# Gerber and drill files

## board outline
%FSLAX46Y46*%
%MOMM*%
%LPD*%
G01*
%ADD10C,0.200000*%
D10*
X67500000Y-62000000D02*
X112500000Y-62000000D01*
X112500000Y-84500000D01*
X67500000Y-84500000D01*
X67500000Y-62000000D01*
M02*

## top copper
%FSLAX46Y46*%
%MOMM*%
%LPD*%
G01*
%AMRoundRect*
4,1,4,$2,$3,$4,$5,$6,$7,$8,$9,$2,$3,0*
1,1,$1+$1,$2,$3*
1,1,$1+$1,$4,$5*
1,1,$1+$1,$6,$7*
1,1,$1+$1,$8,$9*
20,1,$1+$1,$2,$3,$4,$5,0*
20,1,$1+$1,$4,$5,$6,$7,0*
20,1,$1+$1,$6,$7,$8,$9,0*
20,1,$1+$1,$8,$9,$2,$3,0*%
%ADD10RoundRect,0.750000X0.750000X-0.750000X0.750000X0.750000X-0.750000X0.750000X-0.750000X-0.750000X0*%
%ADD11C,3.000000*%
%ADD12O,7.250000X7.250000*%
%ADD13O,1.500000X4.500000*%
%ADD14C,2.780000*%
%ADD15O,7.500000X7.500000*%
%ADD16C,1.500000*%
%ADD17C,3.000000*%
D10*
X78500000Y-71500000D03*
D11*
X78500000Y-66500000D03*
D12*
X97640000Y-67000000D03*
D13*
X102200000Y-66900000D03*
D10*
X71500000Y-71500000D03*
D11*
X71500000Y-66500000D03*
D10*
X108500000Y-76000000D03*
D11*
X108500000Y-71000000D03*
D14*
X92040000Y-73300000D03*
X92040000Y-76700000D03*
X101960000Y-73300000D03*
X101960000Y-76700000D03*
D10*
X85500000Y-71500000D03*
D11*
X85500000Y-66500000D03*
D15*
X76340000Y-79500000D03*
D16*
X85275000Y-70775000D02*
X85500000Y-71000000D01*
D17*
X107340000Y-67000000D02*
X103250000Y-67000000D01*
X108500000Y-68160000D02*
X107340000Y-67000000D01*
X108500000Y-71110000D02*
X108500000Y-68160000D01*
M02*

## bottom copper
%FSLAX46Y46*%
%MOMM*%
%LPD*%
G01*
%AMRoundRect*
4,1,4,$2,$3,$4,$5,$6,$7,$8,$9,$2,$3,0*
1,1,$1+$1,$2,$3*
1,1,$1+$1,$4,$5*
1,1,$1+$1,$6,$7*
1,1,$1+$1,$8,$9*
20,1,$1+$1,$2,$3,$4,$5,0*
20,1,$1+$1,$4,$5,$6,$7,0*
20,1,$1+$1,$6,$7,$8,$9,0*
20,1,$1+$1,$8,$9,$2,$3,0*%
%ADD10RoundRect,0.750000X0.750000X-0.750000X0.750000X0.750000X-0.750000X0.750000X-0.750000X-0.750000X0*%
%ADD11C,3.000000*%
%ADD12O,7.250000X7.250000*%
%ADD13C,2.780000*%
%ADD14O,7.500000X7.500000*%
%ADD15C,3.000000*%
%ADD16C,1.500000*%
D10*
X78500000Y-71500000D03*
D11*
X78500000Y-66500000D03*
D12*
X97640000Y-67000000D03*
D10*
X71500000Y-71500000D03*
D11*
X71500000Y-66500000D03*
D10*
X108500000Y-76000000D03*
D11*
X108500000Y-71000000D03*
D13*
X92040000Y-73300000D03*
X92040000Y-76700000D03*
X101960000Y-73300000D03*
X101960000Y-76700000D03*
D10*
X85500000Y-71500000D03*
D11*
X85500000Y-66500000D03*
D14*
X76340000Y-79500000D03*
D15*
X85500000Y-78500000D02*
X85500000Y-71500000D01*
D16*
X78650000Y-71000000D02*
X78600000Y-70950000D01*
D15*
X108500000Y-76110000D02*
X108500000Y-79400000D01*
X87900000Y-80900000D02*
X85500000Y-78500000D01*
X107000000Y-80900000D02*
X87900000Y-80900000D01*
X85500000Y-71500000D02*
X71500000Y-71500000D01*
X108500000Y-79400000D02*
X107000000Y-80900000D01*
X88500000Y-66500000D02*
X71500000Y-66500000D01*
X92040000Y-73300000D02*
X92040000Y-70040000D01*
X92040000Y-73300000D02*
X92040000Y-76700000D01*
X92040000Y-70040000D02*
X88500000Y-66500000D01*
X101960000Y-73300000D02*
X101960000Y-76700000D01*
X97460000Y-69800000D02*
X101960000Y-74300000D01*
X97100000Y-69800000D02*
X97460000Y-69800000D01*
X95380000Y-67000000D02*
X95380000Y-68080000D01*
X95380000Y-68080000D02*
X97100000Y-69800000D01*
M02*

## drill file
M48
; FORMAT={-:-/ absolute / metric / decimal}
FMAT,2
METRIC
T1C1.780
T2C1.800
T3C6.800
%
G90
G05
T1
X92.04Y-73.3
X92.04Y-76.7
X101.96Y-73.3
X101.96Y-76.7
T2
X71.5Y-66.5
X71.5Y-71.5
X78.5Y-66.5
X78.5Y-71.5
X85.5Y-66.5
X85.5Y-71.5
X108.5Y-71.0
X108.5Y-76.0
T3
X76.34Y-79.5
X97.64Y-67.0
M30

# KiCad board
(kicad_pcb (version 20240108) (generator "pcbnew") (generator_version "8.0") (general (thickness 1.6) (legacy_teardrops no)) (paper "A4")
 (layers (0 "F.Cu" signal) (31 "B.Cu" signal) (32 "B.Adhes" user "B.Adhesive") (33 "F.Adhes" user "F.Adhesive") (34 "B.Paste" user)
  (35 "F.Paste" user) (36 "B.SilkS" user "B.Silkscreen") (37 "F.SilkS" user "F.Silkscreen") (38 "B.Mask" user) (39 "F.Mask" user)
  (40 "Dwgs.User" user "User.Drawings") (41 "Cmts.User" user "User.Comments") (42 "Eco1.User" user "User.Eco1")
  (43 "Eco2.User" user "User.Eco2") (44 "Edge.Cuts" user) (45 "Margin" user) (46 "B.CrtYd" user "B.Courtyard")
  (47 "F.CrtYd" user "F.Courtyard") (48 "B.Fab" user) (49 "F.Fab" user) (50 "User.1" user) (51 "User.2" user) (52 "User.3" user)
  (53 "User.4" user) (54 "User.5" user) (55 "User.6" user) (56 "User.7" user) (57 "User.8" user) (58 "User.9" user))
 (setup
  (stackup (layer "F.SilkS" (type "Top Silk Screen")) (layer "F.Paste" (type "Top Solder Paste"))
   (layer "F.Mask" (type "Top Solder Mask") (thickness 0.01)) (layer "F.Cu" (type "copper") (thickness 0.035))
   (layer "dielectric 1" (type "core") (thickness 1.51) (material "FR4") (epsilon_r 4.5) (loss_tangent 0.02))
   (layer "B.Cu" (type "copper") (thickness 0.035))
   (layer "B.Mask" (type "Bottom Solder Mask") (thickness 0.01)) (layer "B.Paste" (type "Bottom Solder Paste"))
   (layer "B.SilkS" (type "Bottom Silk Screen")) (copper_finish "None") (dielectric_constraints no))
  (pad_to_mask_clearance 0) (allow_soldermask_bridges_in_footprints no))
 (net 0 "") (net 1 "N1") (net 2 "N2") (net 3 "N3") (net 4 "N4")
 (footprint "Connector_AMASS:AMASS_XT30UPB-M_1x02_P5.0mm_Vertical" (layer "F.Cu") (at 78.5 71.5 90)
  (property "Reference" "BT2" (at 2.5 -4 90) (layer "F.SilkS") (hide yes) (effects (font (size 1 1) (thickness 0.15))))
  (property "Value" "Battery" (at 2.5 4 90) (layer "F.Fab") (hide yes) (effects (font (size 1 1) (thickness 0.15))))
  (pad "1" thru_hole roundrect (at 0 0 90) (size 3 3) (drill 1.8) (layers "*.Cu" "*.Mask") (remove_unused_layers no) (roundrect_rratio 0.25)
   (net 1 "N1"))
  (pad "2" thru_hole circle (at 5 0 90) (size 3 3) (drill 1.8) (layers "*.Cu" "*.Mask") (remove_unused_layers no) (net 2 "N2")))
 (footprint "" (layer "F.Cu") (at 97.64 67)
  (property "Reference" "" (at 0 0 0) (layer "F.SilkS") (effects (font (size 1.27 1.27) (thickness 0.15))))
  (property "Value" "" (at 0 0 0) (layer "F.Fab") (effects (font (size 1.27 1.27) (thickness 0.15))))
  (pad "" thru_hole oval (at 0 0 270) (size 7.25 7.25) (drill 6.8) (layers "*.Cu" "*.Mask") (remove_unused_layers no)))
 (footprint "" (layer "F.Cu") (at 102.2 66.9)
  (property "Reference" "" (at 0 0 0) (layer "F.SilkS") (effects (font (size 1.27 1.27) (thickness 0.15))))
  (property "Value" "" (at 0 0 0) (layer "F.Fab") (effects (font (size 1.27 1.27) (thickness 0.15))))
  (pad "2" smd oval (at 0 0) (size 1.5 4.5) (layers "F.Cu" "F.Paste" "F.Mask") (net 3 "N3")))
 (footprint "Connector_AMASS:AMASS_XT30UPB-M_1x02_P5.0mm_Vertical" (layer "F.Cu") (at 71.5 71.5 90)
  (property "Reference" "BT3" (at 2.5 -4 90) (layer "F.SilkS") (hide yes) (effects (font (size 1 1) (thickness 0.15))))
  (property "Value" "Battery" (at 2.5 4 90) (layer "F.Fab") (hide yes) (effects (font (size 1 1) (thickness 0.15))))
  (pad "1" thru_hole roundrect (at 0 0 90) (size 3 3) (drill 1.8) (layers "*.Cu" "*.Mask") (remove_unused_layers no) (roundrect_rratio 0.25)
   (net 1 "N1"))
  (pad "2" thru_hole circle (at 5 0 90) (size 3 3) (drill 1.8) (layers "*.Cu" "*.Mask") (remove_unused_layers no) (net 2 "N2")))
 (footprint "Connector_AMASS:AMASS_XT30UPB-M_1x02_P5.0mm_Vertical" (layer "F.Cu") (at 108.5 76 90)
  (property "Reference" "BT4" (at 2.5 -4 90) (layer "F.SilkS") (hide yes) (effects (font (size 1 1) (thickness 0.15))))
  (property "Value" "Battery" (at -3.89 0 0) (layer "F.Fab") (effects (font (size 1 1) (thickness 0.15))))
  (pad "1" thru_hole roundrect (at 0 0 90) (size 3 3) (drill 1.8) (layers "*.Cu" "*.Mask") (remove_unused_layers no) (roundrect_rratio 0.25)
   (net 1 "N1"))
  (pad "2" thru_hole circle (at 5 0 90) (size 3 3) (drill 1.8) (layers "*.Cu" "*.Mask") (remove_unused_layers no) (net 3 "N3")))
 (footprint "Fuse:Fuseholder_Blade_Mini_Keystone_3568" (layer "F.Cu") (at 92.04 73.3)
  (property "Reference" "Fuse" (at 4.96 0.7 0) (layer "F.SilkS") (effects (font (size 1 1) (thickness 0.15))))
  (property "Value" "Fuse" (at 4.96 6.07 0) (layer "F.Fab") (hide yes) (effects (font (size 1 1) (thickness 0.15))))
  (pad "1" thru_hole circle (at 0 0) (size 2.78 2.78) (drill 1.78) (layers "*.Cu" "*.Mask") (remove_unused_layers no) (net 2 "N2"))
  (pad "1" thru_hole circle (at 0 3.4) (size 2.78 2.78) (drill 1.78) (layers "*.Cu" "*.Mask") (remove_unused_layers no) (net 2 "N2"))
  (pad "2" thru_hole circle (at 9.92 0) (size 2.78 2.78) (drill 1.78) (layers "*.Cu" "*.Mask") (remove_unused_layers no) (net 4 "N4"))
  (pad "2" thru_hole circle (at 9.92 3.4) (size 2.78 2.78) (drill 1.78) (layers "*.Cu" "*.Mask") (remove_unused_layers no) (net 4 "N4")))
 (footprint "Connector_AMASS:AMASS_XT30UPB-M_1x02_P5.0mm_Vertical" (layer "F.Cu") (at 85.5 71.5 90)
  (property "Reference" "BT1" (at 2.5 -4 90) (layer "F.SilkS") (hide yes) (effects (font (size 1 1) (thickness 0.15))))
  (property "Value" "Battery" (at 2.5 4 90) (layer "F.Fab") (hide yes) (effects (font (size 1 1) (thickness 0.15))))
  (pad "1" thru_hole roundrect (at 0 0 90) (size 3 3) (drill 1.8) (layers "*.Cu" "*.Mask") (remove_unused_layers no) (roundrect_rratio 0.25)
   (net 1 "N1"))
  (pad "2" thru_hole circle (at 5 0 90) (size 3 3) (drill 1.8) (layers "*.Cu" "*.Mask") (remove_unused_layers no) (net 2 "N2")))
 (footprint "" (layer "F.Cu") (at 76.34 79.5)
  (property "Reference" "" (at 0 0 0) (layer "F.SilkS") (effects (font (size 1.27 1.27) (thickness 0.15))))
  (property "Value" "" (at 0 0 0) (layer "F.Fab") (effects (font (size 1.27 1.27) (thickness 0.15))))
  (pad "2" thru_hole oval (at 0 0 270) (size 7.5 7.5) (drill 6.8) (layers "*.Cu" "*.Mask") (remove_unused_layers no)))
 (gr_rect (start 67.5 62) (end 112.5 84.5) (stroke (width 0.2) (type default)) (fill none) (layer "Edge.Cuts"))
 (segment (start 85.275 70.775) (end 85.5 71) (width 1.5) (layer "F.Cu") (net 1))
 (segment (start 85.5 78.5) (end 85.5 71.5) (width 3) (layer "B.Cu") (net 1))
 (segment (start 78.65 71) (end 78.6 70.95) (width 1.5) (layer "B.Cu") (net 1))
 (segment (start 108.5 76.11) (end 108.5 79.4) (width 3) (layer "B.Cu") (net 1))
 (segment (start 87.9 80.9) (end 85.5 78.5) (width 3) (layer "B.Cu") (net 1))
 (segment (start 107 80.9) (end 87.9 80.9) (width 3) (layer "B.Cu") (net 1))
 (segment (start 85.5 71.5) (end 71.5 71.5) (width 3) (layer "B.Cu") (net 1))
 (segment (start 108.5 79.4) (end 107 80.9) (width 3) (layer "B.Cu") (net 1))
 (segment (start 88.5 66.5) (end 71.5 66.5) (width 3) (layer "B.Cu") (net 2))
 (segment (start 92.04 73.3) (end 92.04 70.04) (width 3) (layer "B.Cu") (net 2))
 (segment (start 92.04 73.3) (end 92.04 76.7) (width 3) (layer "B.Cu") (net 2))
 (segment (start 92.04 70.04) (end 88.5 66.5) (width 3) (layer "B.Cu") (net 2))
 (segment (start 101.96 73.3) (end 101.96 76.7) (width 3) (layer "B.Cu") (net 4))
 (segment (start 97.46 69.8) (end 101.96 74.3) (width 3) (layer "B.Cu") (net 4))
 (segment (start 97.1 69.8) (end 97.46 69.8) (width 3) (layer "B.Cu") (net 4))
 (segment (start 95.38 67) (end 95.38 68.08) (width 3) (layer "B.Cu") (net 4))
 (segment (start 95.38 68.08) (end 97.1 69.8) (width 3) (layer "B.Cu") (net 4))
 (segment (start 107.34 67) (end 103.25 67) (width 3) (layer "F.Cu") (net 3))
 (segment (start 108.5 68.16) (end 107.34 67) (width 3) (layer "F.Cu") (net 3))
 (segment (start 108.5 71.11) (end 108.5 68.16) (width 3) (layer "F.Cu") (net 3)))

